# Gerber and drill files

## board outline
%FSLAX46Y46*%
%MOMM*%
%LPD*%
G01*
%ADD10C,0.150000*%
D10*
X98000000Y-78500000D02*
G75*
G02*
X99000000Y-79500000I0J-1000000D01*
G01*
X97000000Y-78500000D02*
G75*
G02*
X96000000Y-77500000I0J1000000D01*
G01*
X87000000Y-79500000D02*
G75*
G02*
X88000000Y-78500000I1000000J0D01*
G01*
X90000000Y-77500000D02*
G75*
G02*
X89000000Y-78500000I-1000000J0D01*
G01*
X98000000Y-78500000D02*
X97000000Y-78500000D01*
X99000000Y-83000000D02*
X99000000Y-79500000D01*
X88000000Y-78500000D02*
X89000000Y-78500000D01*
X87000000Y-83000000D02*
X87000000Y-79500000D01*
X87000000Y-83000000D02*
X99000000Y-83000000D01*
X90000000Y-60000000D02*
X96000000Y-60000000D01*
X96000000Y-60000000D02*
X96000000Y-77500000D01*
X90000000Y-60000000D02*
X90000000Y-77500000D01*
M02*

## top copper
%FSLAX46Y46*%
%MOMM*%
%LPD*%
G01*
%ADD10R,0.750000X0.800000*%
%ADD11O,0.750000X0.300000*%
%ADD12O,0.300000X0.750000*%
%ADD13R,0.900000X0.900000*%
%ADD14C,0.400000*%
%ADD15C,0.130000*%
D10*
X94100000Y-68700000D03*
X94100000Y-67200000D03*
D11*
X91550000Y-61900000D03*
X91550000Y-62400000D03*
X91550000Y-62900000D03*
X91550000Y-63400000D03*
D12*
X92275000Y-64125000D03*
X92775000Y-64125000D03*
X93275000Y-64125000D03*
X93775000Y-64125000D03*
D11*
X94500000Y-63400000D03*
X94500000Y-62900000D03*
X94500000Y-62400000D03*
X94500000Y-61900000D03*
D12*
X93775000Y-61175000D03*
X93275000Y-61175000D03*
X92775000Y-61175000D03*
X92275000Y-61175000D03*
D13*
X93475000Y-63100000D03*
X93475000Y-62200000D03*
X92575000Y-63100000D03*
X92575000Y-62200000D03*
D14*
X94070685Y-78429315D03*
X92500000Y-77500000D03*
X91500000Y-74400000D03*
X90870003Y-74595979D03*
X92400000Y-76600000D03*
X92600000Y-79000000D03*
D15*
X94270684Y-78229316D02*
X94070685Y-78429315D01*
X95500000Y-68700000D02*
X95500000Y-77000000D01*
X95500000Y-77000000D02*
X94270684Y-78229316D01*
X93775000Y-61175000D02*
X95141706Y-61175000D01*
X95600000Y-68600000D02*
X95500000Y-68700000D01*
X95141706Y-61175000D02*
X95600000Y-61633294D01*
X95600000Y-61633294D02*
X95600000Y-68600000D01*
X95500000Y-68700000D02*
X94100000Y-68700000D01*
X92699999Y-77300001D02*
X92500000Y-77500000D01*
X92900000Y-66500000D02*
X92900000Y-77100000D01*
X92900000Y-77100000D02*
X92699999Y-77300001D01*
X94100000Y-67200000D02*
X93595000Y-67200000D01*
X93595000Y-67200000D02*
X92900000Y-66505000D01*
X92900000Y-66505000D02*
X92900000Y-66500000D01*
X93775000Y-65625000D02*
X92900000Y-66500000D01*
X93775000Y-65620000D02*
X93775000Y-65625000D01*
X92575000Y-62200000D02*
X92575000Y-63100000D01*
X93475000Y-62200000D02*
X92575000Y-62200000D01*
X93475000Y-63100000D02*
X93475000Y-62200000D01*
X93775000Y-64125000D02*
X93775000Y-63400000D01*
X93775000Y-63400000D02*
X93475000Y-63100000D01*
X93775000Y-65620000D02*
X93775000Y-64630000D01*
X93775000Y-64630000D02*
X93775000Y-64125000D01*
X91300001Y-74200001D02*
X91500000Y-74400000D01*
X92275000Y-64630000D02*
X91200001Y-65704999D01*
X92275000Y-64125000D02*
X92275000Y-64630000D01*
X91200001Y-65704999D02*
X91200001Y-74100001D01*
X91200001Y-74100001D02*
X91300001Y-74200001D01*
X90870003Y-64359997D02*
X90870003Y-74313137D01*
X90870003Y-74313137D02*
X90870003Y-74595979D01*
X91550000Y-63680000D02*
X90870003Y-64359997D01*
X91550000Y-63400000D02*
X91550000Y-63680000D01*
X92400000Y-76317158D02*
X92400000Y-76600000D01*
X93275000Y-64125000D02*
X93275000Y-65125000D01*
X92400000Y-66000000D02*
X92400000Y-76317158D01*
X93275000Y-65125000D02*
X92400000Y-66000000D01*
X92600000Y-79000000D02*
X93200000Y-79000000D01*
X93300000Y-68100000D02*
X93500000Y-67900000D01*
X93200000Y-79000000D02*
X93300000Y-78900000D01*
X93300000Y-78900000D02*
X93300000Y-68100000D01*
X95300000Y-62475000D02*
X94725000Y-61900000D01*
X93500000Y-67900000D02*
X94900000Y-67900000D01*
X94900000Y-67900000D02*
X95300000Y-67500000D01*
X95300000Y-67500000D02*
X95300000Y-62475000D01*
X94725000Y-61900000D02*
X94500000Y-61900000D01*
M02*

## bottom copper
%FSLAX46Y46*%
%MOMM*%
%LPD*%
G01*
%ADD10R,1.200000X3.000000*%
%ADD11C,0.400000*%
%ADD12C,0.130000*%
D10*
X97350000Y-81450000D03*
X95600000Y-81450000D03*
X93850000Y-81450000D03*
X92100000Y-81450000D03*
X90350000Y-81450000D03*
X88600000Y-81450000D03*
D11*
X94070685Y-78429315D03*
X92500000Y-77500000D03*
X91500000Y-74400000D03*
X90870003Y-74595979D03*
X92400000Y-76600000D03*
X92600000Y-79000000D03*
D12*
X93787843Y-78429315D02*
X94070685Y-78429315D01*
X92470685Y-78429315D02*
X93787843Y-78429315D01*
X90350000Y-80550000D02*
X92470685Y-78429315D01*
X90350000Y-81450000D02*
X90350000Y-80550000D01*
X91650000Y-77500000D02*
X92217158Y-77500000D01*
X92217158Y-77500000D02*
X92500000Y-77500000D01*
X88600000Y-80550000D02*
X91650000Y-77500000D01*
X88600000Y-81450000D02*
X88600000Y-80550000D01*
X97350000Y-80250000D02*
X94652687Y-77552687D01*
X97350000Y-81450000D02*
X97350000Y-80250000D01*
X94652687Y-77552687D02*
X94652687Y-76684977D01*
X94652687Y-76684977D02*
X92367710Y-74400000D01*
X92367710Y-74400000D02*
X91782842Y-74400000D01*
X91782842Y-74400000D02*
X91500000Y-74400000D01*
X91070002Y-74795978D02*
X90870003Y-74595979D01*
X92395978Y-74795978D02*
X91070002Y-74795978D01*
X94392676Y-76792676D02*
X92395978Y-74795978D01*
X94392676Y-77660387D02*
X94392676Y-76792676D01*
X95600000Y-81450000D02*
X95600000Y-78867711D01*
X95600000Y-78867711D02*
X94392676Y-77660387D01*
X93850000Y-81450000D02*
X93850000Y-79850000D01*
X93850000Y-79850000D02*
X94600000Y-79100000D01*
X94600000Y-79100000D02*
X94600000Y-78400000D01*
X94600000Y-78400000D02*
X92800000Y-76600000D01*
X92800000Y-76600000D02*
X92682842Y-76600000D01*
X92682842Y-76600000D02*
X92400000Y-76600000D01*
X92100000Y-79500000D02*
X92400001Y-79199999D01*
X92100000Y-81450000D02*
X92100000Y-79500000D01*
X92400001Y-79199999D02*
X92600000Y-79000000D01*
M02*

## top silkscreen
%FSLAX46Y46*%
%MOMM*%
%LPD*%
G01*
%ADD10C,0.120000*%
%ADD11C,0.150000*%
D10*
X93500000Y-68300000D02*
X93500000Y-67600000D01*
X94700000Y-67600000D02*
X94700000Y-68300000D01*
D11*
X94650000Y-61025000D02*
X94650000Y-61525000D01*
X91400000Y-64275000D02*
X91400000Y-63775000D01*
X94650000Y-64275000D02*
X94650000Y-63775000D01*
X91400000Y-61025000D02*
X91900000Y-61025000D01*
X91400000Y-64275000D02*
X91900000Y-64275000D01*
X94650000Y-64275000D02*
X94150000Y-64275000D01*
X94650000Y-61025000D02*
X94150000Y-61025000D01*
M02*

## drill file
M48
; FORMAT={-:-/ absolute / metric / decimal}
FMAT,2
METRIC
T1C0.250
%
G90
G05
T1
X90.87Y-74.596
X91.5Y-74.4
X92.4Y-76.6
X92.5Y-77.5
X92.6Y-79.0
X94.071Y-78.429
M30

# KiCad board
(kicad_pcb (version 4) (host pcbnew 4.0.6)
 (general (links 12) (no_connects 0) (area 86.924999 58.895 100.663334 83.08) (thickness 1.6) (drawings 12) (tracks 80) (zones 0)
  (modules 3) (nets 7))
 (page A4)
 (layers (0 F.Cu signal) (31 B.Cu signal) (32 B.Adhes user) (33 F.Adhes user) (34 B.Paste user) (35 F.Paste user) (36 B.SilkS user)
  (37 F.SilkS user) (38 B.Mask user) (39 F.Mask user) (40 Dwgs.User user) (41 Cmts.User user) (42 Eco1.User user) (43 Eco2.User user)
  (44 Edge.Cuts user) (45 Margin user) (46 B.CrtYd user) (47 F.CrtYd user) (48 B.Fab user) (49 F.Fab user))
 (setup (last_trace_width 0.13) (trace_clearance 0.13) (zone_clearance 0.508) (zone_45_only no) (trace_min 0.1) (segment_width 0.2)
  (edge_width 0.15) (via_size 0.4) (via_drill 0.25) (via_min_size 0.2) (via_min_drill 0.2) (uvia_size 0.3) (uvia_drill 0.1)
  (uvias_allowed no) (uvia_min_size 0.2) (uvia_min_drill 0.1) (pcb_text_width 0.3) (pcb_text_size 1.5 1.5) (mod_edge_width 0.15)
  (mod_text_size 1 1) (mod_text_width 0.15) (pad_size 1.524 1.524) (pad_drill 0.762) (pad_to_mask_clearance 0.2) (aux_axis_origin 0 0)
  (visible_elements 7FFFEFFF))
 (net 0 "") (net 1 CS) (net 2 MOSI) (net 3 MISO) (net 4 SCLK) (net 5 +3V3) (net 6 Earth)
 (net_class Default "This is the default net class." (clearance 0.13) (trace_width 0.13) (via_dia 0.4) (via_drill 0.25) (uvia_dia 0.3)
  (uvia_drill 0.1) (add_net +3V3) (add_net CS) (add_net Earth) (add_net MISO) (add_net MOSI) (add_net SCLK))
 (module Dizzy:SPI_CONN (layer B.Cu) (at 95.7 78.7 180)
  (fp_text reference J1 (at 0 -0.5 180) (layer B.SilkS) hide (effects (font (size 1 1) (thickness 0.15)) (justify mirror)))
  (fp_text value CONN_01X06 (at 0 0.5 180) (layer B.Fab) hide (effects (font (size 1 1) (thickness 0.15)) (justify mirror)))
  (pad 1 smd rect (at -1.65 -2.75 180) (size 1.2 3) (layers B.Cu B.Paste B.Mask) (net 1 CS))
  (pad 2 smd rect (at 0.1 -2.75 180) (size 1.2 3) (layers B.Cu B.Paste B.Mask) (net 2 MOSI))
  (pad 3 smd rect (at 1.85 -2.75 180) (size 1.2 3) (layers B.Cu B.Paste B.Mask) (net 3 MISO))
  (pad 4 smd rect (at 3.6 -2.75 180) (size 1.2 3) (layers B.Cu B.Paste B.Mask) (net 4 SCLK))
  (pad 5 smd rect (at 5.35 -2.75 180) (size 1.2 3) (layers B.Cu B.Paste B.Mask) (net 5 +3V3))
  (pad 6 smd rect (at 7.1 -2.75 180) (size 1.2 3) (layers B.Cu B.Paste B.Mask) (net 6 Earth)))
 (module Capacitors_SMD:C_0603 (layer F.Cu) (at 94.1 67.95 270)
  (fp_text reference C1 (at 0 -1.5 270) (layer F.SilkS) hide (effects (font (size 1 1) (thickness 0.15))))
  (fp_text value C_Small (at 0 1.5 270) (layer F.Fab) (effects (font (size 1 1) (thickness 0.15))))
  (fp_line (start 0.35 0.6) (end -0.35 0.6) (layer F.SilkS) (width 0.12))
  (fp_line (start -0.35 -0.6) (end 0.35 -0.6) (layer F.SilkS) (width 0.12))
  (pad 2 smd rect (at 0.75 0 270) (size 0.8 0.75) (layers F.Cu F.Paste F.Mask) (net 5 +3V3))
  (pad 1 smd rect (at -0.75 0 270) (size 0.8 0.75) (layers F.Cu F.Paste F.Mask) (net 6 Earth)))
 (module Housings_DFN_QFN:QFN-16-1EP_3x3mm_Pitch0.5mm (layer F.Cu) (at 93.025 62.65)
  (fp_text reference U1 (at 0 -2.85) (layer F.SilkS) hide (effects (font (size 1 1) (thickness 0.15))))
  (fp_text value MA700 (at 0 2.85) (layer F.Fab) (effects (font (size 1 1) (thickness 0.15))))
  (fp_line (start 1.625 -1.625) (end 1.625 -1.125) (layer F.SilkS) (width 0.15))
  (fp_line (start -1.625 1.625) (end -1.625 1.125) (layer F.SilkS) (width 0.15))
  (fp_line (start 1.625 1.625) (end 1.625 1.125) (layer F.SilkS) (width 0.15))
  (fp_line (start -1.625 -1.625) (end -1.125 -1.625) (layer F.SilkS) (width 0.15))
  (fp_line (start -1.625 1.625) (end -1.125 1.625) (layer F.SilkS) (width 0.15))
  (fp_line (start 1.625 1.625) (end 1.125 1.625) (layer F.SilkS) (width 0.15))
  (fp_line (start 1.625 -1.625) (end 1.125 -1.625) (layer F.SilkS) (width 0.15))
  (pad 1 smd oval (at -1.475 -0.75) (size 0.75 0.3) (layers F.Cu F.Paste F.Mask))
  (pad 2 smd oval (at -1.475 -0.25) (size 0.75 0.3) (layers F.Cu F.Paste F.Mask))
  (pad 3 smd oval (at -1.475 0.25) (size 0.75 0.3) (layers F.Cu F.Paste F.Mask))
  (pad 4 smd oval (at -1.475 0.75) (size 0.75 0.3) (layers F.Cu F.Paste F.Mask) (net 2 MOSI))
  (pad 5 smd oval (at -0.75 1.475 90) (size 0.75 0.3) (layers F.Cu F.Paste F.Mask) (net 1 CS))
  (pad 6 smd oval (at -0.25 1.475 90) (size 0.75 0.3) (layers F.Cu F.Paste F.Mask))
  (pad 7 smd oval (at 0.25 1.475 90) (size 0.75 0.3) (layers F.Cu F.Paste F.Mask) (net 3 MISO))
  (pad 8 smd oval (at 0.75 1.475 90) (size 0.75 0.3) (layers F.Cu F.Paste F.Mask) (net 6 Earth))
  (pad 9 smd oval (at 1.475 0.75) (size 0.75 0.3) (layers F.Cu F.Paste F.Mask))
  (pad 10 smd oval (at 1.475 0.25) (size 0.75 0.3) (layers F.Cu F.Paste F.Mask))
  (pad 11 smd oval (at 1.475 -0.25) (size 0.75 0.3) (layers F.Cu F.Paste F.Mask))
  (pad 12 smd oval (at 1.475 -0.75) (size 0.75 0.3) (layers F.Cu F.Paste F.Mask) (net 4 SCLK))
  (pad 13 smd oval (at 0.75 -1.475 90) (size 0.75 0.3) (layers F.Cu F.Paste F.Mask) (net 5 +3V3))
  (pad 14 smd oval (at 0.25 -1.475 90) (size 0.75 0.3) (layers F.Cu F.Paste F.Mask))
  (pad 15 smd oval (at -0.25 -1.475 90) (size 0.75 0.3) (layers F.Cu F.Paste F.Mask))
  (pad 16 smd oval (at -0.75 -1.475 90) (size 0.75 0.3) (layers F.Cu F.Paste F.Mask))
  (pad 17 smd rect (at 0.45 0.45) (size 0.9 0.9) (layers F.Cu F.Paste F.Mask) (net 6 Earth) (solder_paste_margin_ratio -0.2))
  (pad 17 smd rect (at 0.45 -0.45) (size 0.9 0.9) (layers F.Cu F.Paste F.Mask) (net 6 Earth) (solder_paste_margin_ratio -0.2))
  (pad 17 smd rect (at -0.45 0.45) (size 0.9 0.9) (layers F.Cu F.Paste F.Mask) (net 6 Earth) (solder_paste_margin_ratio -0.2))
  (pad 17 smd rect (at -0.45 -0.45) (size 0.9 0.9) (layers F.Cu F.Paste F.Mask) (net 6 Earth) (solder_paste_margin_ratio -0.2)))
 (gr_arc (start 98 79.5) (end 98 78.5) (angle 90) (layer Edge.Cuts) (width 0.15))
 (gr_arc (start 97 77.5) (end 97 78.5) (angle 90) (layer Edge.Cuts) (width 0.15))
 (gr_arc (start 88 79.5) (end 87 79.5) (angle 90) (layer Edge.Cuts) (width 0.15))
 (gr_arc (start 89 77.5) (end 90 77.5) (angle 90) (layer Edge.Cuts) (width 0.15))
 (gr_line (start 98 78.5) (end 97 78.5) (layer Edge.Cuts) (width 0.15))
 (gr_line (start 99 83) (end 99 79.5) (layer Edge.Cuts) (width 0.15))
 (gr_line (start 88 78.5) (end 89 78.5) (layer Edge.Cuts) (width 0.15))
 (gr_line (start 87 83) (end 87 79.5) (layer Edge.Cuts) (width 0.15))
 (gr_line (start 87 83) (end 99 83) (layer Edge.Cuts) (width 0.15))
 (gr_line (start 90 60) (end 96 60) (layer Edge.Cuts) (width 0.15))
 (gr_line (start 96 60) (end 96 77.5) (layer Edge.Cuts) (width 0.15))
 (gr_line (start 90 60) (end 90 77.5) (layer Edge.Cuts) (width 0.15))
 (segment (start 94.270684 78.229316) (end 94.070685 78.429315) (width 0.13) (layer F.Cu) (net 5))
 (segment (start 95.5 68.7) (end 95.5 77) (width 0.13) (layer F.Cu) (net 5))
 (segment (start 93.787843 78.429315) (end 94.070685 78.429315) (width 0.13) (layer B.Cu) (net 5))
 (segment (start 92.470685 78.429315) (end 93.787843 78.429315) (width 0.13) (layer B.Cu) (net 5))
 (segment (start 90.35 80.55) (end 92.470685 78.429315) (width 0.13) (layer B.Cu) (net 5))
 (segment (start 95.5 77) (end 94.270684 78.229316) (width 0.13) (layer F.Cu) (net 5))
 (segment (start 90.35 81.45) (end 90.35 80.55) (width 0.13) (layer B.Cu) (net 5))
 (via (at 94.070685 78.429315) (size 0.4) (drill 0.25) (layers F.Cu B.Cu) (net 5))
 (segment (start 93.775 61.175) (end 95.141706 61.175) (width 0.13) (layer F.Cu) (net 5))
 (segment (start 95.6 68.6) (end 95.5 68.7) (width 0.13) (layer F.Cu) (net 5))
 (segment (start 95.141706 61.175) (end 95.6 61.633294) (width 0.13) (layer F.Cu) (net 5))
 (segment (start 95.6 61.633294) (end 95.6 68.6) (width 0.13) (layer F.Cu) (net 5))
 (segment (start 95.5 68.7) (end 94.1 68.7) (width 0.13) (layer F.Cu) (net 5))
 (segment (start 91.65 77.5) (end 92.217158 77.5) (width 0.13) (layer B.Cu) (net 6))
 (segment (start 92.217158 77.5) (end 92.5 77.5) (width 0.13) (layer B.Cu) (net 6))
 (segment (start 88.6 80.55) (end 91.65 77.5) (width 0.13) (layer B.Cu) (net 6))
 (segment (start 88.6 81.45) (end 88.6 80.55) (width 0.13) (layer B.Cu) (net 6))
 (segment (start 92.699999 77.300001) (end 92.5 77.5) (width 0.13) (layer F.Cu) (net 6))
 (segment (start 92.9 66.5) (end 92.9 77.1) (width 0.13) (layer F.Cu) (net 6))
 (segment (start 92.9 77.1) (end 92.699999 77.300001) (width 0.13) (layer F.Cu) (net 6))
 (via (at 92.5 77.5) (size 0.4) (drill 0.25) (layers F.Cu B.Cu) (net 6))
 (segment (start 94.1 67.2) (end 93.595 67.2) (width 0.13) (layer F.Cu) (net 6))
 (segment (start 93.595 67.2) (end 92.9 66.505) (width 0.13) (layer F.Cu) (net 6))
 (segment (start 92.9 66.505) (end 92.9 66.5) (width 0.13) (layer F.Cu) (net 6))
 (segment (start 93.775 65.625) (end 92.9 66.5) (width 0.13) (layer F.Cu) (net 6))
 (segment (start 93.775 65.62) (end 93.775 65.625) (width 0.13) (layer F.Cu) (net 6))
 (segment (start 92.575 62.2) (end 92.575 63.1) (width 0.13) (layer F.Cu) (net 6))
 (segment (start 93.475 62.2) (end 92.575 62.2) (width 0.13) (layer F.Cu) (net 6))
 (segment (start 93.475 63.1) (end 93.475 62.2) (width 0.13) (layer F.Cu) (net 6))
 (segment (start 93.775 64.125) (end 93.775 63.4) (width 0.13) (layer F.Cu) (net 6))
 (segment (start 93.775 63.4) (end 93.475 63.1) (width 0.13) (layer F.Cu) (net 6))
 (segment (start 93.775 65.62) (end 93.775 64.63) (width 0.13) (layer F.Cu) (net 6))
 (segment (start 93.775 64.63) (end 93.775 64.125) (width 0.13) (layer F.Cu) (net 6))
 (segment (start 97.35 80.25) (end 94.652687 77.552687) (width 0.13) (layer B.Cu) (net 1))
 (segment (start 97.35 81.45) (end 97.35 80.25) (width 0.13) (layer B.Cu) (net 1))
 (segment (start 94.652687 77.552687) (end 94.652687 76.684977) (width 0.13) (layer B.Cu) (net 1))
 (segment (start 94.652687 76.684977) (end 92.36771 74.4) (width 0.13) (layer B.Cu) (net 1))
 (segment (start 92.36771 74.4) (end 91.782842 74.4) (width 0.13) (layer B.Cu) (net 1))
 (segment (start 91.782842 74.4) (end 91.5 74.4) (width 0.13) (layer B.Cu) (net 1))
 (segment (start 91.300001 74.200001) (end 91.5 74.4) (width 0.13) (layer F.Cu) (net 1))
 (segment (start 92.275 64.63) (end 91.200001 65.704999) (width 0.13) (layer F.Cu) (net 1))
 (segment (start 92.275 64.125) (end 92.275 64.63) (width 0.13) (layer F.Cu) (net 1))
 (segment (start 91.200001 65.704999) (end 91.200001 74.100001) (width 0.13) (layer F.Cu) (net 1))
 (via (at 91.5 74.4) (size 0.4) (drill 0.25) (layers F.Cu B.Cu) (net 1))
 (segment (start 91.200001 74.100001) (end 91.300001 74.200001) (width 0.13) (layer F.Cu) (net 1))
 (segment (start 91.070002 74.795978) (end 90.870003 74.595979) (width 0.13) (layer B.Cu) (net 2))
 (segment (start 92.395978 74.795978) (end 91.070002 74.795978) (width 0.13) (layer B.Cu) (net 2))
 (segment (start 94.392676 76.792676) (end 92.395978 74.795978) (width 0.13) (layer B.Cu) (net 2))
 (segment (start 94.392676 77.660387) (end 94.392676 76.792676) (width 0.13) (layer B.Cu) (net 2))
 (segment (start 95.6 81.45) (end 95.6 78.867711) (width 0.13) (layer B.Cu) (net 2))
 (segment (start 95.6 78.867711) (end 94.392676 77.660387) (width 0.13) (layer B.Cu) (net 2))
 (segment (start 90.870003 64.359997) (end 90.870003 74.313137) (width 0.13) (layer F.Cu) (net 2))
 (segment (start 90.870003 74.313137) (end 90.870003 74.595979) (width 0.13) (layer F.Cu) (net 2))
 (via (at 90.870003 74.595979) (size 0.4) (drill 0.25) (layers F.Cu B.Cu) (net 2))
 (segment (start 91.55 63.68) (end 90.870003 64.359997) (width 0.13) (layer F.Cu) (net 2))
 (segment (start 91.55 63.4) (end 91.55 63.68) (width 0.13) (layer F.Cu) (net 2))
 (segment (start 93.85 81.45) (end 93.85 79.85) (width 0.13) (layer B.Cu) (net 3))
 (segment (start 93.85 79.85) (end 94.6 79.1) (width 0.13) (layer B.Cu) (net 3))
 (segment (start 94.6 79.1) (end 94.6 78.4) (width 0.13) (layer B.Cu) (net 3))
 (segment (start 94.6 78.4) (end 92.8 76.6) (width 0.13) (layer B.Cu) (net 3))
 (segment (start 92.8 76.6) (end 92.682842 76.6) (width 0.13) (layer B.Cu) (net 3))
 (segment (start 92.682842 76.6) (end 92.4 76.6) (width 0.13) (layer B.Cu) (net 3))
 (via (at 92.4 76.6) (size 0.4) (drill 0.25) (layers F.Cu B.Cu) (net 3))
 (segment (start 92.4 76.317158) (end 92.4 76.6) (width 0.13) (layer F.Cu) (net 3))
 (segment (start 93.275 64.125) (end 93.275 65.125) (width 0.13) (layer F.Cu) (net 3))
 (segment (start 92.4 66) (end 92.4 76.317158) (width 0.13) (layer F.Cu) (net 3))
 (segment (start 93.275 65.125) (end 92.4 66) (width 0.13) (layer F.Cu) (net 3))
 (segment (start 92.6 79) (end 93.2 79) (width 0.13) (layer F.Cu) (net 4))
 (segment (start 93.3 68.1) (end 93.5 67.9) (width 0.13) (layer F.Cu) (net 4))
 (segment (start 93.2 79) (end 93.3 78.9) (width 0.13) (layer F.Cu) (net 4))
 (segment (start 93.3 78.9) (end 93.3 68.1) (width 0.13) (layer F.Cu) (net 4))
 (segment (start 95.3 62.475) (end 94.725 61.9) (width 0.13) (layer F.Cu) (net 4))
 (segment (start 93.5 67.9) (end 94.9 67.9) (width 0.13) (layer F.Cu) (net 4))
 (segment (start 94.9 67.9) (end 95.3 67.5) (width 0.13) (layer F.Cu) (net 4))
 (segment (start 95.3 67.5) (end 95.3 62.475) (width 0.13) (layer F.Cu) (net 4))
 (segment (start 94.725 61.9) (end 94.5 61.9) (width 0.13) (layer F.Cu) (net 4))
 (segment (start 92.1 79.5) (end 92.400001 79.199999) (width 0.13) (layer B.Cu) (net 4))
 (segment (start 92.1 81.45) (end 92.1 79.5) (width 0.13) (layer B.Cu) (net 4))
 (segment (start 92.400001 79.199999) (end 92.6 79) (width 0.13) (layer B.Cu) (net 4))
 (via (at 92.6 79) (size 0.4) (drill 0.25) (layers F.Cu B.Cu) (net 4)))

